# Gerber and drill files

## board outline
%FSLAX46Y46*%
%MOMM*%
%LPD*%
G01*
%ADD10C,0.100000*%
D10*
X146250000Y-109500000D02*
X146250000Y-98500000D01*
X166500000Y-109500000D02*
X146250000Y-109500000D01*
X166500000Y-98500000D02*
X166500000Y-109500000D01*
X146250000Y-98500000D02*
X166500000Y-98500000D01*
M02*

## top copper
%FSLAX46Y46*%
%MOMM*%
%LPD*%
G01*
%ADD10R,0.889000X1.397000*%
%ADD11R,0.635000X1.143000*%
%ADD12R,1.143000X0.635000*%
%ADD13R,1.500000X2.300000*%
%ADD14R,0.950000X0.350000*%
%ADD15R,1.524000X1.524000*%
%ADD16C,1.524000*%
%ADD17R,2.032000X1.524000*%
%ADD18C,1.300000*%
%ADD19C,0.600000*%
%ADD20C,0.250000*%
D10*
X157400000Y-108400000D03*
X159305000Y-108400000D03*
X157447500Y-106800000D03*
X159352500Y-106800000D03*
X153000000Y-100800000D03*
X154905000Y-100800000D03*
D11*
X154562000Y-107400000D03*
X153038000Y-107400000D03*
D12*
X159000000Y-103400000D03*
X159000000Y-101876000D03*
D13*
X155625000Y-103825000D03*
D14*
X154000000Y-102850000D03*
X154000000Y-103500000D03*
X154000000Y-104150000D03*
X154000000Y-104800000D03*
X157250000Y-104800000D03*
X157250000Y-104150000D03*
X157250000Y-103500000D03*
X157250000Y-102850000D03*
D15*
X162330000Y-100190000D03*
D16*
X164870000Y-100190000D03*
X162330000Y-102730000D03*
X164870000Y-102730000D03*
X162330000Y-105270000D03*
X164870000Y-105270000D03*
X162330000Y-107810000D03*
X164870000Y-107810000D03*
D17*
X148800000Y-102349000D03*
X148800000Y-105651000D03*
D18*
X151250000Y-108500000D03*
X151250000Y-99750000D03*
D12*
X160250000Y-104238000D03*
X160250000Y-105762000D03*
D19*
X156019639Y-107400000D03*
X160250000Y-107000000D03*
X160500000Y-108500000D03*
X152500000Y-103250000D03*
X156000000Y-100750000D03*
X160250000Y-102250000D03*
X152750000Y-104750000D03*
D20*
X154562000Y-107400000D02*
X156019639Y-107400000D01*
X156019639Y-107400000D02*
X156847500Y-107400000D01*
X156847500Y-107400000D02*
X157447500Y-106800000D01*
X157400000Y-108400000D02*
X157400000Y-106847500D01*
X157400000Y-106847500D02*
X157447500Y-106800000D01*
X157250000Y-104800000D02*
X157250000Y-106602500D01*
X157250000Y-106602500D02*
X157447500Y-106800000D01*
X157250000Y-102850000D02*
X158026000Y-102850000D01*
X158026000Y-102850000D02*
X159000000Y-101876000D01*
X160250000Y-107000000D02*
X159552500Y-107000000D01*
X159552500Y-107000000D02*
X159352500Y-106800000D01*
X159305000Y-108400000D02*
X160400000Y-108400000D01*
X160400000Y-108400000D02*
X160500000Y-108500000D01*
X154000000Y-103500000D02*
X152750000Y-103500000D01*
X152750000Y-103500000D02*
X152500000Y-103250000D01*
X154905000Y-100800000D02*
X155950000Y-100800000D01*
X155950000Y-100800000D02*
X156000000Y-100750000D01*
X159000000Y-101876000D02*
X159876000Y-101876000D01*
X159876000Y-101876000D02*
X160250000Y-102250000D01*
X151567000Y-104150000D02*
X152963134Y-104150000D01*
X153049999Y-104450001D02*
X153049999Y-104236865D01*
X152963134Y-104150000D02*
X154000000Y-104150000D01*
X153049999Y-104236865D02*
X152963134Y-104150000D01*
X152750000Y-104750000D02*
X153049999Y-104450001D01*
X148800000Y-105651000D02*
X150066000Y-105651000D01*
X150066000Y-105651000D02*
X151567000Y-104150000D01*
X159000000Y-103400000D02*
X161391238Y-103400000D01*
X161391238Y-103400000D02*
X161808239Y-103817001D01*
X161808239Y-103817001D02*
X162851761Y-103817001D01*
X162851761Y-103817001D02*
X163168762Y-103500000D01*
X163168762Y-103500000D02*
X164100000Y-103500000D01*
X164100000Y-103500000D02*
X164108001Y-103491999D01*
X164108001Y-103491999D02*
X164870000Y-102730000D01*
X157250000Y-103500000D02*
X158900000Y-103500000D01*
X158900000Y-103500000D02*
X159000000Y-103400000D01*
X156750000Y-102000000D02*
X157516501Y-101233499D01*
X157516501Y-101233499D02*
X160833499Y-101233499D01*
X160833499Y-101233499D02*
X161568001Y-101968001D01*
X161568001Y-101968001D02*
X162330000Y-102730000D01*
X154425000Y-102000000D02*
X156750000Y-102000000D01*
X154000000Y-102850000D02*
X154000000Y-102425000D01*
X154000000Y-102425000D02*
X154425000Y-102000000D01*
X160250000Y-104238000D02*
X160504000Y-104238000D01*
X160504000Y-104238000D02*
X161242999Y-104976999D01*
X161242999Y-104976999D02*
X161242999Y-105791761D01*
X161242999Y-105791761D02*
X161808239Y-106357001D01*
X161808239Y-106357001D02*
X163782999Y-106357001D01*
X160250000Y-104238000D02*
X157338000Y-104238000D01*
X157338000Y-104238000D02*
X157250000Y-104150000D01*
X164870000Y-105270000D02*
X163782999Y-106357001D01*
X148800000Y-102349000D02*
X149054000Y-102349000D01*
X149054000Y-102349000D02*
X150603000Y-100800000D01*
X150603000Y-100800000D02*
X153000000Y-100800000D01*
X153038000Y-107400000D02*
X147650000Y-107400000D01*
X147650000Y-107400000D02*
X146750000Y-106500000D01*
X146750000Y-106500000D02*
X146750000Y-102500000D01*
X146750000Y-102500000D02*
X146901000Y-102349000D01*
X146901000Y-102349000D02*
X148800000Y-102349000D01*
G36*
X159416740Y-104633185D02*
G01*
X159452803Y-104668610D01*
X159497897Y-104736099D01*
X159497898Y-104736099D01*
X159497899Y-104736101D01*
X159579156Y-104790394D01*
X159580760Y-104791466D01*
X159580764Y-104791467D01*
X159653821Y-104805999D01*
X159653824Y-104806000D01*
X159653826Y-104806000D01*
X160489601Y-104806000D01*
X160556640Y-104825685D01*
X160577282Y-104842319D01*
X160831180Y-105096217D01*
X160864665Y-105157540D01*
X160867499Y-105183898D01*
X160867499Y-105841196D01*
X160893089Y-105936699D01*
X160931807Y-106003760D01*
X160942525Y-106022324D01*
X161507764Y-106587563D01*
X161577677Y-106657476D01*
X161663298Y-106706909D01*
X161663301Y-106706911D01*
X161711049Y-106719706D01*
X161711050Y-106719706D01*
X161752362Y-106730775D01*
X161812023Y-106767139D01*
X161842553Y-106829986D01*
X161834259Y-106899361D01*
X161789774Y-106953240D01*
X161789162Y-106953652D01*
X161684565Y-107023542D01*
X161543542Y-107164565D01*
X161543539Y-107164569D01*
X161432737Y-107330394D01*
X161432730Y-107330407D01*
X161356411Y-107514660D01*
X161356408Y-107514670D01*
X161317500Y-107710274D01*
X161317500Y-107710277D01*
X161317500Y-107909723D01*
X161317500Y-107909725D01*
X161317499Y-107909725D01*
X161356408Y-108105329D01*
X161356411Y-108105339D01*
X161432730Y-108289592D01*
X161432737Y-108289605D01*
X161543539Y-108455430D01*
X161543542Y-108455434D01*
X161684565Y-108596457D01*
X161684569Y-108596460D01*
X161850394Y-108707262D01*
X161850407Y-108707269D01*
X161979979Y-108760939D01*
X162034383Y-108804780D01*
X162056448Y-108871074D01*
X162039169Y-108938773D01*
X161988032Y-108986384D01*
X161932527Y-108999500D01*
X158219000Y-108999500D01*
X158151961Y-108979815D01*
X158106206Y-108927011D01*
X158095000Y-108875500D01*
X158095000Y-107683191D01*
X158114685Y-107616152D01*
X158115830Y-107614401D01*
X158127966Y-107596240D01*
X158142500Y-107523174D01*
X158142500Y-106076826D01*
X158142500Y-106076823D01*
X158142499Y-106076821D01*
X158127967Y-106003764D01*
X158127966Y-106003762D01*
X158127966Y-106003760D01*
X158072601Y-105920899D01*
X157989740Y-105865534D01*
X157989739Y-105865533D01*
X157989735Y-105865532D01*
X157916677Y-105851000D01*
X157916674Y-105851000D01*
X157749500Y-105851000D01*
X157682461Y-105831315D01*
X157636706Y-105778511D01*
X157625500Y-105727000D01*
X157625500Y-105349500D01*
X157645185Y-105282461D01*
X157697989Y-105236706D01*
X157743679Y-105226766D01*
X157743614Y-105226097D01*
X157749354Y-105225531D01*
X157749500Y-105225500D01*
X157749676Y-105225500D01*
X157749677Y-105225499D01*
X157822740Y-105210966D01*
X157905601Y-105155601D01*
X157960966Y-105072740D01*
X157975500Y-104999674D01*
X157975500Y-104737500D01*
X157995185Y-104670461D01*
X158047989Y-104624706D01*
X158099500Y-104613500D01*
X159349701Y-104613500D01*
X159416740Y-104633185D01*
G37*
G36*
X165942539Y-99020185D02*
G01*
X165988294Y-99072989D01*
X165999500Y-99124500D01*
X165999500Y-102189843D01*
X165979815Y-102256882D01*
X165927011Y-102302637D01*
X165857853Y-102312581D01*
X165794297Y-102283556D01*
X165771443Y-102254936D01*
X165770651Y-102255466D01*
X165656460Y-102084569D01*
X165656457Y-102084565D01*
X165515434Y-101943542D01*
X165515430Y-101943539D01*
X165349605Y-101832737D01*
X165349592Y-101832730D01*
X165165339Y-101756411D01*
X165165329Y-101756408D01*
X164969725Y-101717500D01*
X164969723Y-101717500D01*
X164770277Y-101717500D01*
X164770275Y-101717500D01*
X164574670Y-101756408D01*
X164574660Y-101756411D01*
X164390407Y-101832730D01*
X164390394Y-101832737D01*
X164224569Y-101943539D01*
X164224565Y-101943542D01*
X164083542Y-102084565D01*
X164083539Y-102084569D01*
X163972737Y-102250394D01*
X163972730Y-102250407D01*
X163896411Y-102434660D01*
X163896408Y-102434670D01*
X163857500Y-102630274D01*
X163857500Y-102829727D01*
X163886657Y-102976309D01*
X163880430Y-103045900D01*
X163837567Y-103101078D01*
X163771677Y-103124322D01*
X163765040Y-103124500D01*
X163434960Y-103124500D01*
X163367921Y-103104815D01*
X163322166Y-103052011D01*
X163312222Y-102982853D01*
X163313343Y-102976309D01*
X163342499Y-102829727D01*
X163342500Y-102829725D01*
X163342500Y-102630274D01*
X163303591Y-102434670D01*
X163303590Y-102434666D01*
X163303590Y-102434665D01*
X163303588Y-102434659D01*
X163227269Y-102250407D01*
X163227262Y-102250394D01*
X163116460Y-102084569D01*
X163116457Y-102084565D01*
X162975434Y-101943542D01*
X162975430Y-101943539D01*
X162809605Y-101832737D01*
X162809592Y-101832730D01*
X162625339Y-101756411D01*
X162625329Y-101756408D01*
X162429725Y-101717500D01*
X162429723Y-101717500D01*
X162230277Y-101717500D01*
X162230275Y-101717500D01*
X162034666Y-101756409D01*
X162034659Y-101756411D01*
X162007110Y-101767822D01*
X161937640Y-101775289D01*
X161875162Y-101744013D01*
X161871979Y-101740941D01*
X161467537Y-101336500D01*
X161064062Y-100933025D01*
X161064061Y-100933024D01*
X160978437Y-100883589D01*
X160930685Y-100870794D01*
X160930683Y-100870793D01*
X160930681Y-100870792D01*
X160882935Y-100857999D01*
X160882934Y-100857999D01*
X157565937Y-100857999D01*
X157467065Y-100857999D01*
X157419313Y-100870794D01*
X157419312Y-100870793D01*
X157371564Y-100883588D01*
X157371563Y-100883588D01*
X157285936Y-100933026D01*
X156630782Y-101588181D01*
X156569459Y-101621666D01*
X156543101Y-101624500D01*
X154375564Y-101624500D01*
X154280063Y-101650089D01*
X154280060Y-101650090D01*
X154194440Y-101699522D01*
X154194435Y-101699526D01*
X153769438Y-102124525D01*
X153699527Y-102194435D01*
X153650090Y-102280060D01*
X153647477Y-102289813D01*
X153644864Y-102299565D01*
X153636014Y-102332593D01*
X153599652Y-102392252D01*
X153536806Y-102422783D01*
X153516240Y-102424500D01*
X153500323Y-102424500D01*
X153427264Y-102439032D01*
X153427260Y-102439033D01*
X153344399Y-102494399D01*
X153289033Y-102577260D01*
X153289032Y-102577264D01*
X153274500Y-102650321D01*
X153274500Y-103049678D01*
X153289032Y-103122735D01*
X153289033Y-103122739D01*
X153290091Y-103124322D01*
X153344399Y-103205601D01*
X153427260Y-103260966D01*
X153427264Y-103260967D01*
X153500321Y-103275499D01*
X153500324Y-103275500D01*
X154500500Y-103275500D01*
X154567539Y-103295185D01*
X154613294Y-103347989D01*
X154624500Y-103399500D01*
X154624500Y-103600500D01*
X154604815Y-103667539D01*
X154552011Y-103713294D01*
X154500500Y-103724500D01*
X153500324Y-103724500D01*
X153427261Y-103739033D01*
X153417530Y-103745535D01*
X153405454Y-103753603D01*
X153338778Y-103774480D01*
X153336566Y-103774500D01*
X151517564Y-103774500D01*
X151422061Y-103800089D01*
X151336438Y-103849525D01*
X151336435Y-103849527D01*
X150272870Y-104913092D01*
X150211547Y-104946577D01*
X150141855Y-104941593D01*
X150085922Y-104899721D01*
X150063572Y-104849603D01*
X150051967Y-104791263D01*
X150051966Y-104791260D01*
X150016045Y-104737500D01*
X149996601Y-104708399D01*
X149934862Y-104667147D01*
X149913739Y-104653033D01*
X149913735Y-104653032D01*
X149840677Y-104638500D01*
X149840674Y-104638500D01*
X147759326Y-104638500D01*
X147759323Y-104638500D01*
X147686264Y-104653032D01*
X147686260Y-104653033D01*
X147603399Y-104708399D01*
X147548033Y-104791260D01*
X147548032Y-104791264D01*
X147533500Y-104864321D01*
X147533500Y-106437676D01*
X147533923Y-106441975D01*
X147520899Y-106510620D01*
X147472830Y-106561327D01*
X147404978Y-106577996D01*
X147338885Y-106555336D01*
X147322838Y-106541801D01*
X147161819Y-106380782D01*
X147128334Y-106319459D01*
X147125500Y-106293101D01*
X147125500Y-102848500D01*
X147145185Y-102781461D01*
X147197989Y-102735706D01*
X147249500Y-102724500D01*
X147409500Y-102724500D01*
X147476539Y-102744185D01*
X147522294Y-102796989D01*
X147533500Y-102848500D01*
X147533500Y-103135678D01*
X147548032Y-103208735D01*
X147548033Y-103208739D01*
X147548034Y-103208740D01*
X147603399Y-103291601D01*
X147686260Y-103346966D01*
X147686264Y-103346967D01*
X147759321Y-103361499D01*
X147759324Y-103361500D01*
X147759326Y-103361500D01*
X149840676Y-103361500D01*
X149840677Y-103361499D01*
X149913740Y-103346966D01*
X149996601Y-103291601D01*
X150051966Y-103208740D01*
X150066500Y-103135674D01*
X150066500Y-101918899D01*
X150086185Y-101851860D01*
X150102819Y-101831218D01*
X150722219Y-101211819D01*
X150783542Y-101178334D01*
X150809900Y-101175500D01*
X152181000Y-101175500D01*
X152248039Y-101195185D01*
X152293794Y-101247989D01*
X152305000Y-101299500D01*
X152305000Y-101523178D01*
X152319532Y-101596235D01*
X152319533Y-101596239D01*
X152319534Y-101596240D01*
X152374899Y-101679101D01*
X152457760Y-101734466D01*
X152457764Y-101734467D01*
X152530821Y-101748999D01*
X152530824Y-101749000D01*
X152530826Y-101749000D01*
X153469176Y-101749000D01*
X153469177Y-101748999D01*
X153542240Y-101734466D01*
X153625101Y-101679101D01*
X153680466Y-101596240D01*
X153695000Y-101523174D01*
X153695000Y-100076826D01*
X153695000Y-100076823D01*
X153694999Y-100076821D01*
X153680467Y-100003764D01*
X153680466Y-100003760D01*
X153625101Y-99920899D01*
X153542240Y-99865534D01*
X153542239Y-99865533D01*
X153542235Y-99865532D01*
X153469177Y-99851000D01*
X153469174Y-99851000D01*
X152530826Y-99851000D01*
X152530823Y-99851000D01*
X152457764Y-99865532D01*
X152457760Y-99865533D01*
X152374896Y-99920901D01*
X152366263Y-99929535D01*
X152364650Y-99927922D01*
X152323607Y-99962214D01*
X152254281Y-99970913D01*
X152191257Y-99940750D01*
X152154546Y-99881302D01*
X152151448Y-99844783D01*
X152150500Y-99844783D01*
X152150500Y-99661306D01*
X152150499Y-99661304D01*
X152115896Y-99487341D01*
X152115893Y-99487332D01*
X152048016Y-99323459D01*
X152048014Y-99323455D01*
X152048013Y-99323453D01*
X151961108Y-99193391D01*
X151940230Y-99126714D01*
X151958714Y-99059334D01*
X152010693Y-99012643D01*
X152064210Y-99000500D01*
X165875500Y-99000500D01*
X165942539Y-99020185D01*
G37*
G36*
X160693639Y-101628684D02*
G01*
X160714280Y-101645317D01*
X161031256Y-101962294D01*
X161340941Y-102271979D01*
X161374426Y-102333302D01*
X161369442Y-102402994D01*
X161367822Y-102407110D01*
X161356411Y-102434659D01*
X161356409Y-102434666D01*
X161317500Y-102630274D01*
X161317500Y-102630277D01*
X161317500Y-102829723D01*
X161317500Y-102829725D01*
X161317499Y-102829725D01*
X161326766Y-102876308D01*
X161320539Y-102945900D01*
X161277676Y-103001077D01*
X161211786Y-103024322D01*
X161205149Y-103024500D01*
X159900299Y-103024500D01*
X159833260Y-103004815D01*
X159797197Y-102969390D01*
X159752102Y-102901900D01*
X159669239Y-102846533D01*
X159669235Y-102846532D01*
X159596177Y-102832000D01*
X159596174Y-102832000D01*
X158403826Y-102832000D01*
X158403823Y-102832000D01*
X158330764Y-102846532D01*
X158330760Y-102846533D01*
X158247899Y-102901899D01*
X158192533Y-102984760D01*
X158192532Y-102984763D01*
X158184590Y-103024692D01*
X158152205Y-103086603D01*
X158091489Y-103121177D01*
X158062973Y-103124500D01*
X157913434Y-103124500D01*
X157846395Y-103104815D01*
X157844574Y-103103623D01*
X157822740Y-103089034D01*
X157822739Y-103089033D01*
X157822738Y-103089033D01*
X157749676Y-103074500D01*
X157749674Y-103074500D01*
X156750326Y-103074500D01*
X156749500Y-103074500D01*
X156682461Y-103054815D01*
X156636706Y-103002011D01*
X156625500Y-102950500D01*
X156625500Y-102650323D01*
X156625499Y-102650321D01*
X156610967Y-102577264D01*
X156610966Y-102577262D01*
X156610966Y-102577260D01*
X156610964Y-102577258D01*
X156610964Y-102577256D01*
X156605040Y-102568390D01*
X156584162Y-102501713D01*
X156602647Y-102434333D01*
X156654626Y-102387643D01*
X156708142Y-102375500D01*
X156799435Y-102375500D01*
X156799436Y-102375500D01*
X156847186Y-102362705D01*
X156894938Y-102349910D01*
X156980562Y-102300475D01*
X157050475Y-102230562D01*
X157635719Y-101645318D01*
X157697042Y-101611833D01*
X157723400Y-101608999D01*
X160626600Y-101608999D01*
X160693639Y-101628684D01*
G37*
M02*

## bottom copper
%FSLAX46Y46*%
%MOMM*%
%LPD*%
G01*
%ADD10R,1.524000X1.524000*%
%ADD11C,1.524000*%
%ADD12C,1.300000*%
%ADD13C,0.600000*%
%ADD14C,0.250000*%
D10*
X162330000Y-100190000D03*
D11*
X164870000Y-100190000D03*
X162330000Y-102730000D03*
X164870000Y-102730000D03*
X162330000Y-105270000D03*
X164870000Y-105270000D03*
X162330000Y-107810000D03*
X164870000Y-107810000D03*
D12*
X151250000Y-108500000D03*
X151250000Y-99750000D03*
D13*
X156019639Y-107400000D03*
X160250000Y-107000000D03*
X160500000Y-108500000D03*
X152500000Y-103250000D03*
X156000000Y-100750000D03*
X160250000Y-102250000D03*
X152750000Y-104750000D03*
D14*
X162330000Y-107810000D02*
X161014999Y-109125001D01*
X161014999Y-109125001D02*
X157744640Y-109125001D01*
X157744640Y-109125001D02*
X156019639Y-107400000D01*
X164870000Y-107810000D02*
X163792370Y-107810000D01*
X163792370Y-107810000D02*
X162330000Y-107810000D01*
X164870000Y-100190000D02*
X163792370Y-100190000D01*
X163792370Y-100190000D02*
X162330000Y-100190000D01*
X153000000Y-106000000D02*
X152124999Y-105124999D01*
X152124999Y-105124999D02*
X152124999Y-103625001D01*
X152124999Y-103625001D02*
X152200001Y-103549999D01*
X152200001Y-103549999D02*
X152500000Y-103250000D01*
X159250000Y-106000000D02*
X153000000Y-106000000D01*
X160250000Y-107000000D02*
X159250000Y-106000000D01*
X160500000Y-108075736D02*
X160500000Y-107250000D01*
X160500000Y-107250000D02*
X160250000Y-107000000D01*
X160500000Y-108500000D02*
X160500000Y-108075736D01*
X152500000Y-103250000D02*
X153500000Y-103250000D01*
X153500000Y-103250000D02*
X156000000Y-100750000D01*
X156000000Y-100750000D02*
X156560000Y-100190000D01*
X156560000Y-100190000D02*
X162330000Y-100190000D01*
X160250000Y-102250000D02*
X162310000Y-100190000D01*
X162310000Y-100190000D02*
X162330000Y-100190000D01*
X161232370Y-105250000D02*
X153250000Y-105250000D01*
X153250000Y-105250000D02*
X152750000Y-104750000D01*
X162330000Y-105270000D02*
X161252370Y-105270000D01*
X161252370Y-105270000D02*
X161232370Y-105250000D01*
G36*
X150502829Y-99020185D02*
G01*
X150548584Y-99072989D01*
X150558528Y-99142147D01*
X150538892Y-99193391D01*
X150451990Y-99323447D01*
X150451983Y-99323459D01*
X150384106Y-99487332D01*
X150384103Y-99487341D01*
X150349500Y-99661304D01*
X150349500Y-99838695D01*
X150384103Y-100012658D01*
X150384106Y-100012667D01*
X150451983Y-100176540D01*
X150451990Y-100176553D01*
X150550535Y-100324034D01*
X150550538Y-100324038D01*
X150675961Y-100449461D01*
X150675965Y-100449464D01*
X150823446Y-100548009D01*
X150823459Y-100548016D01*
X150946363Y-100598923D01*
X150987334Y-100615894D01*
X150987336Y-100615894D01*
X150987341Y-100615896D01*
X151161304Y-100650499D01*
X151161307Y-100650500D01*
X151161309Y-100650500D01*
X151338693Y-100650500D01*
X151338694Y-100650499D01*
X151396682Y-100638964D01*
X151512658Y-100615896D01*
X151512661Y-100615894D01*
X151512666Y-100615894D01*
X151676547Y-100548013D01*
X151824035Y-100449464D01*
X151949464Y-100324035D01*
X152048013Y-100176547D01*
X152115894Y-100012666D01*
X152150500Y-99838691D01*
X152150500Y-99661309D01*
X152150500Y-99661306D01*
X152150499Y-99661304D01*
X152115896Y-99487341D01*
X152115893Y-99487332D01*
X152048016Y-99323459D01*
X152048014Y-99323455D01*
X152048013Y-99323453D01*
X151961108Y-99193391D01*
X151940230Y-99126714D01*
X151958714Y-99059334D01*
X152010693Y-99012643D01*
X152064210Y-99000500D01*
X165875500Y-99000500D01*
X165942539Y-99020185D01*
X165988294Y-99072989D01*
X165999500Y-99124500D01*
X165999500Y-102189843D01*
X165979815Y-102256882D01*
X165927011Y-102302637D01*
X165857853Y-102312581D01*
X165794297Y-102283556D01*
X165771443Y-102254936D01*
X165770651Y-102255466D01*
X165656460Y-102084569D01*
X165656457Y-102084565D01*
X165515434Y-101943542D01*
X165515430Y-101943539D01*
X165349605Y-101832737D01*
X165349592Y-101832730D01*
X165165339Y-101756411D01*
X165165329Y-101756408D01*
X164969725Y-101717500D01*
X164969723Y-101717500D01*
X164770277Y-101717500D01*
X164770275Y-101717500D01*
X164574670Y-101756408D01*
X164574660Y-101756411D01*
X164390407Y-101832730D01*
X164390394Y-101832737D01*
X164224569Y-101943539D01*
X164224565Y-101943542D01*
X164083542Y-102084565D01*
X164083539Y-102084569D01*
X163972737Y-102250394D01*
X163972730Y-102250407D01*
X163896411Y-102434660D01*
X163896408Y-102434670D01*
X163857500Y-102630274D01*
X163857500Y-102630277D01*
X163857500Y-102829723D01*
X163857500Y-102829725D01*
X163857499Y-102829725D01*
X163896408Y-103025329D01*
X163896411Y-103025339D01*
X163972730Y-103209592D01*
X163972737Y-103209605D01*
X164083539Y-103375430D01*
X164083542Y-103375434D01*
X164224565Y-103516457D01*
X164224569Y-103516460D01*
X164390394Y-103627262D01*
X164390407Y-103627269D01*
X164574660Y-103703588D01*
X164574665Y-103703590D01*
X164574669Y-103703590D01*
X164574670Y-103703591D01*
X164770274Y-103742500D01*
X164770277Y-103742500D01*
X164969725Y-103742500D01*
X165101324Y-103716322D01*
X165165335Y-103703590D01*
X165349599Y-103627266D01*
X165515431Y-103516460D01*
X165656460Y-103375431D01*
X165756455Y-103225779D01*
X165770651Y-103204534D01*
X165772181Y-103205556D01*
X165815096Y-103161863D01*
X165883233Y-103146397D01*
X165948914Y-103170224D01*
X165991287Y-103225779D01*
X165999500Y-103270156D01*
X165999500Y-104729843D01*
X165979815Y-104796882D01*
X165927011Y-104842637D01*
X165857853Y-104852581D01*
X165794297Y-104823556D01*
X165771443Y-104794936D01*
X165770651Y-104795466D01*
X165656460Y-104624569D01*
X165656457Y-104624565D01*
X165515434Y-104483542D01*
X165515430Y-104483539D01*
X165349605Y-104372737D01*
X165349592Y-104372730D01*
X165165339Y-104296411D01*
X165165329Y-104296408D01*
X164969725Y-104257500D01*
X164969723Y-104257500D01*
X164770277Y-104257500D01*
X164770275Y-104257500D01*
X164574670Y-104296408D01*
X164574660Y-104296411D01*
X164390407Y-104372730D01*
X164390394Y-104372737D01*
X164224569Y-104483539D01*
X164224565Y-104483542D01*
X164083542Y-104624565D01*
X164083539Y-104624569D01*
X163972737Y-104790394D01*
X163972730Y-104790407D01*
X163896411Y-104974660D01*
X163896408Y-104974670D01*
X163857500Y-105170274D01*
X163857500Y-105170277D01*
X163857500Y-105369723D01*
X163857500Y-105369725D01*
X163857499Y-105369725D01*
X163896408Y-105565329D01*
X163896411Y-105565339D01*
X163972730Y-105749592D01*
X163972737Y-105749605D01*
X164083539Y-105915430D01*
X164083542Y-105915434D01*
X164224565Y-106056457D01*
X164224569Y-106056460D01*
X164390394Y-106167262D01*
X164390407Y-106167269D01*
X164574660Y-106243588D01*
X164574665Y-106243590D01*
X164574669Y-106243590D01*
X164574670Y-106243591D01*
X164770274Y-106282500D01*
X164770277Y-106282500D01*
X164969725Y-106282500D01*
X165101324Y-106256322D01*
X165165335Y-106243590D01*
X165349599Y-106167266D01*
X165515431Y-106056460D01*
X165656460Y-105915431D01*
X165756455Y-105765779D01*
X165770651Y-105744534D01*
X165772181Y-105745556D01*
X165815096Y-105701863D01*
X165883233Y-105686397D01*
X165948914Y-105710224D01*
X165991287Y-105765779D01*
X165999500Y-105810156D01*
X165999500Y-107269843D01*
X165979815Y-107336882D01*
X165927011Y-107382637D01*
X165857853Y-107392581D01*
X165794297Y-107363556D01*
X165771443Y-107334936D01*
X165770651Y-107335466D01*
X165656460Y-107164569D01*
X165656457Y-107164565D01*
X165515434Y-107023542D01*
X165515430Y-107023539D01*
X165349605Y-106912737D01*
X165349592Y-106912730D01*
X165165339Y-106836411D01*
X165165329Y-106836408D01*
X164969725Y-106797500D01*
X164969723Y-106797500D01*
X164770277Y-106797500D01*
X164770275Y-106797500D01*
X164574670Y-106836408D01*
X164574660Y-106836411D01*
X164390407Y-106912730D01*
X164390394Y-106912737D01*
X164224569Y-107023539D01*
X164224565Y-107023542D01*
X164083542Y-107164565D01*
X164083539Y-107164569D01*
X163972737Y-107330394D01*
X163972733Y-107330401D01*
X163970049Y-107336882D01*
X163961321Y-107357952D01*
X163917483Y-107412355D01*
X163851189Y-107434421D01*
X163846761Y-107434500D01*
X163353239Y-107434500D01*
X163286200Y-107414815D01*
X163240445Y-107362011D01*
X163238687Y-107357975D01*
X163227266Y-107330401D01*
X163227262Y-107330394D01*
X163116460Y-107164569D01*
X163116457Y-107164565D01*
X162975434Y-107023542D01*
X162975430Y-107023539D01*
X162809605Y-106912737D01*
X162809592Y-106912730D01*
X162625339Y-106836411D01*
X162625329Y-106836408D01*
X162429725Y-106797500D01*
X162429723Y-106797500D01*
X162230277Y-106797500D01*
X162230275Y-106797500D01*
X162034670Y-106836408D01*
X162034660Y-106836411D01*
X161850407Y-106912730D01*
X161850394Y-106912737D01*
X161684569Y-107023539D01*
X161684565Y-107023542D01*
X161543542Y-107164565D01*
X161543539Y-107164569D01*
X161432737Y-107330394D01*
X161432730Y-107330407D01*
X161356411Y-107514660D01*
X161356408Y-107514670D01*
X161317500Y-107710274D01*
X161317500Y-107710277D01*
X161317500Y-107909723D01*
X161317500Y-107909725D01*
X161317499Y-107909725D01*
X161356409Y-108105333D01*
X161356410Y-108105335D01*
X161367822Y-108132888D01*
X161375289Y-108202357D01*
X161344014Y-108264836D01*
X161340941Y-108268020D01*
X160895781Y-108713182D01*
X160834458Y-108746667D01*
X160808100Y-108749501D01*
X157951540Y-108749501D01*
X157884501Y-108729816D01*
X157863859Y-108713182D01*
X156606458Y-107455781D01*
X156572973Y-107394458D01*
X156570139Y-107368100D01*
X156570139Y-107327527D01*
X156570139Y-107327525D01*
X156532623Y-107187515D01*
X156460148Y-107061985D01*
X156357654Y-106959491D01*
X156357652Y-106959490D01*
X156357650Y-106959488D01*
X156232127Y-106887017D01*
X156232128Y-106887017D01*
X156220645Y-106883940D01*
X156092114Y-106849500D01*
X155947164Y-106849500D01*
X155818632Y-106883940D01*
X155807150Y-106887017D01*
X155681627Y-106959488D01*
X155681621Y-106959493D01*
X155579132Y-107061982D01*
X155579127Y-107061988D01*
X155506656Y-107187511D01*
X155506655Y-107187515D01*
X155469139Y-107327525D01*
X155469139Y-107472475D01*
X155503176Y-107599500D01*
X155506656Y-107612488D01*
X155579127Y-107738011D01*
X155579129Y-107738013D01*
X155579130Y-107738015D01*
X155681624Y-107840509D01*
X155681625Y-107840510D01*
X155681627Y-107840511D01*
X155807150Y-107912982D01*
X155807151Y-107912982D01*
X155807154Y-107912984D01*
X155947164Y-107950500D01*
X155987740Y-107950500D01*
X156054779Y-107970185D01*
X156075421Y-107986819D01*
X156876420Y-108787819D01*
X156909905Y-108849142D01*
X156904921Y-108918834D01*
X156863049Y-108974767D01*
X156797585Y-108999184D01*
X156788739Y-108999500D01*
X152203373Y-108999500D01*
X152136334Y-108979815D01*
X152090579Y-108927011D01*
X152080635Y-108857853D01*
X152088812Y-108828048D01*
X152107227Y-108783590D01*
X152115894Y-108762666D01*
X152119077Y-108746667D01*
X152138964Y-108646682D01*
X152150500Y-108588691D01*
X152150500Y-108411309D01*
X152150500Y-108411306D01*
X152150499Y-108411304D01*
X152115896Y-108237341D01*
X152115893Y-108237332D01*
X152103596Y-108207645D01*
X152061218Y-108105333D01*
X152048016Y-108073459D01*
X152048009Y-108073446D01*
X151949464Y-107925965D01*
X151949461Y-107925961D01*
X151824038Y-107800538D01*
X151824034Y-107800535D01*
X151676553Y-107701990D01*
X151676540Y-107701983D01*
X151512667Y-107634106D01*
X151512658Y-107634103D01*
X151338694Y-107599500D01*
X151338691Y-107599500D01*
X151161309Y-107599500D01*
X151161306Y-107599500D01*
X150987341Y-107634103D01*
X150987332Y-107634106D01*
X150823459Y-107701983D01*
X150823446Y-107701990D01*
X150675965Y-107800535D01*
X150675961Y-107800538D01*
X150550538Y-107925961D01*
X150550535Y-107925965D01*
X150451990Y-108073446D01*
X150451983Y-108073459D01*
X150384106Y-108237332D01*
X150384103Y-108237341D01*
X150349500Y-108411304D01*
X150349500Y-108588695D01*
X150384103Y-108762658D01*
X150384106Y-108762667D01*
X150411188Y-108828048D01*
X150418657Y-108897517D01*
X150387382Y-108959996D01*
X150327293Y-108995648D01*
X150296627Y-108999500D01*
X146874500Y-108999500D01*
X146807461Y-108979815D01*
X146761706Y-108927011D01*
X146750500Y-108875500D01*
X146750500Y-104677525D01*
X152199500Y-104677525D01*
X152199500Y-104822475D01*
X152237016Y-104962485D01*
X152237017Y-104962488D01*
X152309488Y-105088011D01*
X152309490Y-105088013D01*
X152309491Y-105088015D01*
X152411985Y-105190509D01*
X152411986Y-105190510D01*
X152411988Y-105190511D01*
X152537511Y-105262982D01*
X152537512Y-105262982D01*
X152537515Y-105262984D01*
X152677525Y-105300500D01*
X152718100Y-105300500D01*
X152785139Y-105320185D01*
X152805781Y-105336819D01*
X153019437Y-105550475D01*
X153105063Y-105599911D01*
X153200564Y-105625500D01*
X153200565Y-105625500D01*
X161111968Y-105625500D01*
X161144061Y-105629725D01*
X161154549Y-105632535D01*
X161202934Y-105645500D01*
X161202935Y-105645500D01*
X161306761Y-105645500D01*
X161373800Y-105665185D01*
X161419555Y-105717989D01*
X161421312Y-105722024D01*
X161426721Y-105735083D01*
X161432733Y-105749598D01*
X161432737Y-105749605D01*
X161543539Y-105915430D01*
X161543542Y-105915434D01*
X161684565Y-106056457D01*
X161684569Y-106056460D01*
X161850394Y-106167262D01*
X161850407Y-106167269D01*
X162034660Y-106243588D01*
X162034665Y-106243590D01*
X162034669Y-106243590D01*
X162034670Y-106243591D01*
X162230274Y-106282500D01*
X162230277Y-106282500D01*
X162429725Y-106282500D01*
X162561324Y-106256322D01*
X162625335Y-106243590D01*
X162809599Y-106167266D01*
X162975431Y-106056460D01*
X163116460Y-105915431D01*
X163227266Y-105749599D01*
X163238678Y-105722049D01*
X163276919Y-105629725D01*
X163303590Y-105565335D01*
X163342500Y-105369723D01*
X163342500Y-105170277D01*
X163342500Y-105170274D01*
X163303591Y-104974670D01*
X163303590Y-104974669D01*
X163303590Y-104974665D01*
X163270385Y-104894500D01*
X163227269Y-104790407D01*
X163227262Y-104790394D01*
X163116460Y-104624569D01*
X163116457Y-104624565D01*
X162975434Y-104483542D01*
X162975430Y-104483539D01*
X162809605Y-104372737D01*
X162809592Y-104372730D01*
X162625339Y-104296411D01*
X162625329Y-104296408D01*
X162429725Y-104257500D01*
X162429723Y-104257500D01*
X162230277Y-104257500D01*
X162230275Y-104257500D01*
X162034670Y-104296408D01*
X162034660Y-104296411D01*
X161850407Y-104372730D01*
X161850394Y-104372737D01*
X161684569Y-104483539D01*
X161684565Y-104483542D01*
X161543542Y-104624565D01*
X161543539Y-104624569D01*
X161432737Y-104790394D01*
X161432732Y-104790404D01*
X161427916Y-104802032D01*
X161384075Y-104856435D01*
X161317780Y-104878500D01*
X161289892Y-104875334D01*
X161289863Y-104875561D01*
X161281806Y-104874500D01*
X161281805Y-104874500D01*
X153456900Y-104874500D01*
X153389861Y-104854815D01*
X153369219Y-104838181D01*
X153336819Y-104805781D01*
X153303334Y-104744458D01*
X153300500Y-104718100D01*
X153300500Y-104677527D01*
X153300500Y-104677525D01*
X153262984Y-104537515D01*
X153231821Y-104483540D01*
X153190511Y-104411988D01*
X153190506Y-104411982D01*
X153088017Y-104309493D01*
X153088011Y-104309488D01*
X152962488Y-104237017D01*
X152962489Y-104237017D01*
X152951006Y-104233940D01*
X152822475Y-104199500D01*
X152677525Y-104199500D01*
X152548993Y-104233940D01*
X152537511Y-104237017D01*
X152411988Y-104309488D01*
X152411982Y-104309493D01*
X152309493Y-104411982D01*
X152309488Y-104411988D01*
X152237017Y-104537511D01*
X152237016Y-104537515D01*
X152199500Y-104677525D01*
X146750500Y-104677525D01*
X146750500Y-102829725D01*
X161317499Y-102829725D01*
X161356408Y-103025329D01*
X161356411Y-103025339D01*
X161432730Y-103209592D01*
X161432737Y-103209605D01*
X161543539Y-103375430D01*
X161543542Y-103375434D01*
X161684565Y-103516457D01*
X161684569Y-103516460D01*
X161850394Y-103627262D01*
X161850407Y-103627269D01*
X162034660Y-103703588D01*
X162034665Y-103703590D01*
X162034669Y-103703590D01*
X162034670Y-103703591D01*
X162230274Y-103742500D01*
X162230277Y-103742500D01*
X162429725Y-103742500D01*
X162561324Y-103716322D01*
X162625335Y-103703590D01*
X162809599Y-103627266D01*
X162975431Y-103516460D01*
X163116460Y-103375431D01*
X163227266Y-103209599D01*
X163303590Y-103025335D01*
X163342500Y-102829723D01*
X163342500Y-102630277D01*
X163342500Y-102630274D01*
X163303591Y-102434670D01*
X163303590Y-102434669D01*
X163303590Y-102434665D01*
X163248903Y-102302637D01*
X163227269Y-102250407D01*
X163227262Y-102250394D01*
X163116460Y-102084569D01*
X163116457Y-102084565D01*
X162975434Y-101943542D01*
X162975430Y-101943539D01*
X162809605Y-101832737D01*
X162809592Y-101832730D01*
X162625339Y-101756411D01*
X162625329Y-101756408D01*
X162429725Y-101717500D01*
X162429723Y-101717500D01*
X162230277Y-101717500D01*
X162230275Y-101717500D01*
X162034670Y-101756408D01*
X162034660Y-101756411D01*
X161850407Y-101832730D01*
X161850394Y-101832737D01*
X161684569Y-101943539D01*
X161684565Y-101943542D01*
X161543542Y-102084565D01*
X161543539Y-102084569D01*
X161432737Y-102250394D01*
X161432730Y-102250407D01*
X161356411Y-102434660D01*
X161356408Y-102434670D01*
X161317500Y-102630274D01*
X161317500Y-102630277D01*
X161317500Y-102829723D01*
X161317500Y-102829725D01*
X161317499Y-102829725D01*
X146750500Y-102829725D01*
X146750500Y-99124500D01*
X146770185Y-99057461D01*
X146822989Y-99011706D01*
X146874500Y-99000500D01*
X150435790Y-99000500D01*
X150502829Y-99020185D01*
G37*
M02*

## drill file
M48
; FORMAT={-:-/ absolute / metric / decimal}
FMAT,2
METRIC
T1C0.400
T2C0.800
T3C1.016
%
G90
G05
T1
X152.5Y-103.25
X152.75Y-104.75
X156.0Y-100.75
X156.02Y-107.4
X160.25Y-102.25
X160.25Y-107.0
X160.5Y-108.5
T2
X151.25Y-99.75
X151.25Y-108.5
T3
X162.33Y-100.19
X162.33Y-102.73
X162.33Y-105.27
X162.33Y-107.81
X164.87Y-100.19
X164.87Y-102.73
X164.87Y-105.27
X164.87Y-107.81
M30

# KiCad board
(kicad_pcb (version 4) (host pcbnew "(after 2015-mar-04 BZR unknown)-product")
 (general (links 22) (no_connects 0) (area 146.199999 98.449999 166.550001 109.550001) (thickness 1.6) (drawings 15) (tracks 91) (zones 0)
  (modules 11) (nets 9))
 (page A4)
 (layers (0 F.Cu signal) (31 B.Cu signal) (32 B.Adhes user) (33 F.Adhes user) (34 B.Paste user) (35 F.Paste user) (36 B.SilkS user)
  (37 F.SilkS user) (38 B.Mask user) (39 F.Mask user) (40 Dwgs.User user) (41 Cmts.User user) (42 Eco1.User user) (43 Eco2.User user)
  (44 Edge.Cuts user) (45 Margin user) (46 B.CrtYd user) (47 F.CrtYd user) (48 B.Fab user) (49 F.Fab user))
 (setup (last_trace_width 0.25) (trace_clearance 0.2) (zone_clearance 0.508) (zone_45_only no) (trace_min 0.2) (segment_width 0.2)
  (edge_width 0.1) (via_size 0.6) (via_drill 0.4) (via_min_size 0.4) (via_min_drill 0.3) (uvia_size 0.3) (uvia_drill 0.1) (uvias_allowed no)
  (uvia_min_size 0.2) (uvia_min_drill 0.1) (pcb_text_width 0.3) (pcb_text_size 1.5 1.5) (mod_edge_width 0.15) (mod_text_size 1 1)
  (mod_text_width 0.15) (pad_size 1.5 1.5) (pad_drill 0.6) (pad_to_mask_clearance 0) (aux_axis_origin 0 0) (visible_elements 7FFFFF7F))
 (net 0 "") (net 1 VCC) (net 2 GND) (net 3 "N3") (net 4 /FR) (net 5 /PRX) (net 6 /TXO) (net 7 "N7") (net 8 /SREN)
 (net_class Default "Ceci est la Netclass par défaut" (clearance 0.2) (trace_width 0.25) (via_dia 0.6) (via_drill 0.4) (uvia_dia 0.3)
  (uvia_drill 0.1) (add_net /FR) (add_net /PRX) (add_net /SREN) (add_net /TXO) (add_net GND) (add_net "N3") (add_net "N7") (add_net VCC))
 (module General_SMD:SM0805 (layer F.Cu) (at 158.3525 108.4)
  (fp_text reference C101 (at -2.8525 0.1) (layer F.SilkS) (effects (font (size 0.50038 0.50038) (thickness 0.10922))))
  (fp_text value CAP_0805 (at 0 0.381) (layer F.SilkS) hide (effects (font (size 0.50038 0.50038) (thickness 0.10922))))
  (pad 1 smd rect (at -0.9525 0) (size 0.889 1.397) (layers F.Cu F.Paste F.Mask) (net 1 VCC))
  (pad 2 smd rect (at 0.9525 0) (size 0.889 1.397) (layers F.Cu F.Paste F.Mask) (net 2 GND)))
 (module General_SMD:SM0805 (layer F.Cu) (at 158.4 106.8)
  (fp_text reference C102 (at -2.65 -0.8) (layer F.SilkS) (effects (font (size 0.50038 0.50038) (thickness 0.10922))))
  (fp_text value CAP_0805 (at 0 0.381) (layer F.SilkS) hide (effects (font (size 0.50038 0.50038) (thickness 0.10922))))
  (pad 1 smd rect (at -0.9525 0) (size 0.889 1.397) (layers F.Cu F.Paste F.Mask) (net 1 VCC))
  (pad 2 smd rect (at 0.9525 0) (size 0.889 1.397) (layers F.Cu F.Paste F.Mask) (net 2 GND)))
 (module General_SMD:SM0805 (layer F.Cu) (at 153.9525 100.8)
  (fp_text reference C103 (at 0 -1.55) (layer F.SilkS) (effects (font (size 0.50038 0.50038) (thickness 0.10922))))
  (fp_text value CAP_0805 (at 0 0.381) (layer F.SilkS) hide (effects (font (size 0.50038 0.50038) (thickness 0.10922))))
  (pad 1 smd rect (at -0.9525 0) (size 0.889 1.397) (layers F.Cu F.Paste F.Mask) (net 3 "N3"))
  (pad 2 smd rect (at 0.9525 0) (size 0.889 1.397) (layers F.Cu F.Paste F.Mask) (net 2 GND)))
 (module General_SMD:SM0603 (layer F.Cu) (at 153.8 107.4 180)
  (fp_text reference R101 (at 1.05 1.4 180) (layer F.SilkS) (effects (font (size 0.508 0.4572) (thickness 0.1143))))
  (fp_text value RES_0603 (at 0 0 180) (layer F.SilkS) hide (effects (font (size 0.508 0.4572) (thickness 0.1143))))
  (pad 1 smd rect (at -0.762 0 180) (size 0.635 1.143) (layers F.Cu F.Paste F.Mask) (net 1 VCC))
  (pad 2 smd rect (at 0.762 0 180) (size 0.635 1.143) (layers F.Cu F.Paste F.Mask) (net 3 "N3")))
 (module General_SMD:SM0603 (layer F.Cu) (at 159 102.638 90)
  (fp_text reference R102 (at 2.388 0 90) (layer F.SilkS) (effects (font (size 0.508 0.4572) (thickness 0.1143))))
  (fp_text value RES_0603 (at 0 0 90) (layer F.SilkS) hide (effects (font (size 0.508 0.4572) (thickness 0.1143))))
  (pad 1 smd rect (at -0.762 0 90) (size 0.635 1.143) (layers F.Cu F.Paste F.Mask) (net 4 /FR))
  (pad 2 smd rect (at 0.762 0 90) (size 0.635 1.143) (layers F.Cu F.Paste F.Mask) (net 2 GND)))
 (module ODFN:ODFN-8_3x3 (layer F.Cu) (at 155.625 103.825 270)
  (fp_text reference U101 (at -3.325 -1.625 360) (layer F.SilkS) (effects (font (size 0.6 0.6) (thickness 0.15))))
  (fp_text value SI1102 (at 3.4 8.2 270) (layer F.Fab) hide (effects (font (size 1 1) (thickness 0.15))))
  (pad 9 smd rect (at 0 0 270) (size 2.3 1.5) (layers F.Cu F.Paste F.Mask))
  (pad 1 smd rect (at -0.975 1.625 270) (size 0.35 0.95) (layers F.Cu F.Paste F.Mask) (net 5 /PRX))
  (pad 2 smd rect (at -0.325 1.625 270) (size 0.35 0.95) (layers F.Cu F.Paste F.Mask) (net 2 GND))
  (pad 3 smd rect (at 0.325 1.625 270) (size 0.35 0.95) (layers F.Cu F.Paste F.Mask) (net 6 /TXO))
  (pad 4 smd rect (at 0.975 1.625 270) (size 0.35 0.95) (layers F.Cu F.Paste F.Mask) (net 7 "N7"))
  (pad 5 smd rect (at 0.975 -1.625 270) (size 0.35 0.95) (layers F.Cu F.Paste F.Mask) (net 1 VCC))
  (pad 6 smd rect (at 0.325 -1.625 270) (size 0.35 0.95) (layers F.Cu F.Paste F.Mask) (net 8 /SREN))
  (pad 7 smd rect (at -0.325 -1.625 270) (size 0.35 0.95) (layers F.Cu F.Paste F.Mask) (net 4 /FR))
  (pad 8 smd rect (at -0.975 -1.625 270) (size 0.35 0.95) (layers F.Cu F.Paste F.Mask) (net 2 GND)))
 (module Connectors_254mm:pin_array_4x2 (layer F.Cu) (at 163.6 104 270)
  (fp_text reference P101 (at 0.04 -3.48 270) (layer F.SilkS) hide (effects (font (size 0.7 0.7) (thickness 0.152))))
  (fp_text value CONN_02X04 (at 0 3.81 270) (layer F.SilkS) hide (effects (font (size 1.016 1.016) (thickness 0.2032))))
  (pad 1 thru_hole rect (at -3.81 1.27 270) (size 1.524 1.524) (drill 1.016) (layers *.Cu *.Mask F.SilkS) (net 2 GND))
  (pad 2 thru_hole circle (at -3.81 -1.27 270) (size 1.524 1.524) (drill 1.016) (layers *.Cu *.Mask F.SilkS) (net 2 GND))
  (pad 3 thru_hole circle (at -1.27 1.27 270) (size 1.524 1.524) (drill 1.016) (layers *.Cu *.Mask F.SilkS) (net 5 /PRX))
  (pad 4 thru_hole circle (at -1.27 -1.27 270) (size 1.524 1.524) (drill 1.016) (layers *.Cu *.Mask F.SilkS) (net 4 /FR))
  (pad 5 thru_hole circle (at 1.27 1.27 270) (size 1.524 1.524) (drill 1.016) (layers *.Cu *.Mask F.SilkS) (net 6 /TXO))
  (pad 6 thru_hole circle (at 1.27 -1.27 270) (size 1.524 1.524) (drill 1.016) (layers *.Cu *.Mask F.SilkS) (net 8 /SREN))
  (pad 7 thru_hole circle (at 3.81 1.27 270) (size 1.524 1.524) (drill 1.016) (layers *.Cu *.Mask F.SilkS) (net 1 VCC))
  (pad 8 thru_hole circle (at 3.81 -1.27 270) (size 1.524 1.524) (drill 1.016) (layers *.Cu *.Mask F.SilkS) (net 1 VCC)))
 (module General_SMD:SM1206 (layer F.Cu) (at 148.8 104 270)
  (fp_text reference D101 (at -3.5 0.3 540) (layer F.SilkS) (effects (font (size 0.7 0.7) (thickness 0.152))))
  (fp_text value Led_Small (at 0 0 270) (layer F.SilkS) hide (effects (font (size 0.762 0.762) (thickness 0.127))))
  (pad 1 smd rect (at -1.651 0 270) (size 1.524 2.032) (layers F.Cu F.Paste F.Mask) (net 3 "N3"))
  (pad 2 smd rect (at 1.651 0 270) (size 1.524 2.032) (layers F.Cu F.Paste F.Mask) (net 6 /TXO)))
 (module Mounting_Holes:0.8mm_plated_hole (layer F.Cu) (at 151.25 108.5)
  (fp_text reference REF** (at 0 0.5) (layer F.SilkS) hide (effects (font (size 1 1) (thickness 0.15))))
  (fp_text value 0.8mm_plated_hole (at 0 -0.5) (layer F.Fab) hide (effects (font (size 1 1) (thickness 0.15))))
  (pad 1 thru_hole circle (at 0 0) (size 1.3 1.3) (drill 0.8) (layers *.Cu *.SilkS *.Mask)))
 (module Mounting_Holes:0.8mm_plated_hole (layer F.Cu) (at 151.25 99.75)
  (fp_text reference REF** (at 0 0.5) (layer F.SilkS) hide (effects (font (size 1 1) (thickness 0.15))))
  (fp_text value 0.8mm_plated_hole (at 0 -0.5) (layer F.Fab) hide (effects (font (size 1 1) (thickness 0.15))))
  (pad 1 thru_hole circle (at 0 0) (size 1.3 1.3) (drill 0.8) (layers *.Cu *.SilkS *.Mask)))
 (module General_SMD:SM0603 (layer F.Cu) (at 160.25 105 270)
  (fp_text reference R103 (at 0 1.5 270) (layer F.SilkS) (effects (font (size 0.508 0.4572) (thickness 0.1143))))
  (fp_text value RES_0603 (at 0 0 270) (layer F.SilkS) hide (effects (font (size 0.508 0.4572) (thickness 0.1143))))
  (pad 1 smd rect (at -0.762 0 270) (size 0.635 1.143) (layers F.Cu F.Paste F.Mask) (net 8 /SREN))
  (pad 2 smd rect (at 0.762 0 270) (size 0.635 1.143) (layers F.Cu F.Paste F.Mask) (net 2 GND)))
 (gr_line (start 146.25 109.5) (end 146.25 98.5) (layer Edge.Cuts) (width 0.1))
 (gr_line (start 166.5 109.5) (end 146.25 109.5) (layer Edge.Cuts) (width 0.1))
 (gr_line (start 166.5 98.5) (end 166.5 109.5) (layer Edge.Cuts) (width 0.1))
 (gr_line (start 146.25 98.5) (end 166.5 98.5) (layer Edge.Cuts) (width 0.1))
 (segment (start 154.562 107.4) (end 156.019639 107.4) (width 0.25) (layer F.Cu) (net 1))
 (segment (start 156.019639 107.4) (end 156.8475 107.4) (width 0.25) (layer F.Cu) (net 1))
 (via (at 156.019639 107.4) (size 0.6) (drill 0.4) (layers F.Cu B.Cu) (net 1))
 (segment (start 162.33 107.81) (end 161.014999 109.125001) (width 0.25) (layer B.Cu) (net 1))
 (segment (start 161.014999 109.125001) (end 157.74464 109.125001) (width 0.25) (layer B.Cu) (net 1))
 (segment (start 157.74464 109.125001) (end 156.019639 107.4) (width 0.25) (layer B.Cu) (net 1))
 (segment (start 164.87 107.81) (end 163.79237 107.81) (width 0.25) (layer B.Cu) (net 1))
 (segment (start 163.79237 107.81) (end 162.33 107.81) (width 0.25) (layer B.Cu) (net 1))
 (segment (start 156.8475 107.4) (end 157.4475 106.8) (width 0.25) (layer F.Cu) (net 1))
 (segment (start 157.4 108.4) (end 157.4 106.8475) (width 0.25) (layer F.Cu) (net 1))
 (segment (start 157.4 106.8475) (end 157.4475 106.8) (width 0.25) (layer F.Cu) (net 1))
 (segment (start 157.25 104.8) (end 157.25 106.6025) (width 0.25) (layer F.Cu) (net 1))
 (segment (start 157.25 106.6025) (end 157.4475 106.8) (width 0.25) (layer F.Cu) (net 1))
 (segment (start 164.87 100.19) (end 163.79237 100.19) (width 0.25) (layer B.Cu) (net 2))
 (segment (start 163.79237 100.19) (end 162.33 100.19) (width 0.25) (layer B.Cu) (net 2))
 (segment (start 153 106) (end 152.124999 105.124999) (width 0.25) (layer B.Cu) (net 2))
 (segment (start 152.124999 105.124999) (end 152.124999 103.625001) (width 0.25) (layer B.Cu) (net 2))
 (segment (start 152.124999 103.625001) (end 152.200001 103.549999) (width 0.25) (layer B.Cu) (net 2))
 (segment (start 152.200001 103.549999) (end 152.5 103.25) (width 0.25) (layer B.Cu) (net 2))
 (segment (start 159.25 106) (end 153 106) (width 0.25) (layer B.Cu) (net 2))
 (segment (start 160.25 107) (end 159.25 106) (width 0.25) (layer B.Cu) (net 2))
 (segment (start 157.25 102.85) (end 158.026 102.85) (width 0.25) (layer F.Cu) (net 2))
 (segment (start 158.026 102.85) (end 159 101.876) (width 0.25) (layer F.Cu) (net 2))
 (segment (start 160.25 107) (end 159.5525 107) (width 0.25) (layer F.Cu) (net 2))
 (segment (start 159.5525 107) (end 159.3525 106.8) (width 0.25) (layer F.Cu) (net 2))
 (segment (start 160.5 108.075736) (end 160.5 107.25) (width 0.25) (layer B.Cu) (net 2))
 (segment (start 160.5 107.25) (end 160.25 107) (width 0.25) (layer B.Cu) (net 2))
 (via (at 160.25 107) (size 0.6) (drill 0.4) (layers F.Cu B.Cu) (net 2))
 (segment (start 160.5 108.5) (end 160.5 108.075736) (width 0.25) (layer B.Cu) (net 2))
 (segment (start 159.305 108.4) (end 160.4 108.4) (width 0.25) (layer F.Cu) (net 2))
 (segment (start 160.4 108.4) (end 160.5 108.5) (width 0.25) (layer F.Cu) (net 2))
 (via (at 160.5 108.5) (size 0.6) (drill 0.4) (layers F.Cu B.Cu) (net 2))
 (segment (start 152.5 103.25) (end 153.5 103.25) (width 0.25) (layer B.Cu) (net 2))
 (segment (start 153.5 103.25) (end 156 100.75) (width 0.25) (layer B.Cu) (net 2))
 (segment (start 156 100.75) (end 156.56 100.19) (width 0.25) (layer B.Cu) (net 2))
 (segment (start 156.56 100.19) (end 162.33 100.19) (width 0.25) (layer B.Cu) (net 2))
 (segment (start 160.25 102.25) (end 162.31 100.19) (width 0.25) (layer B.Cu) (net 2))
 (segment (start 162.31 100.19) (end 162.33 100.19) (width 0.25) (layer B.Cu) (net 2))
 (segment (start 154 103.5) (end 152.75 103.5) (width 0.25) (layer F.Cu) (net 2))
 (segment (start 152.75 103.5) (end 152.5 103.25) (width 0.25) (layer F.Cu) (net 2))
 (via (at 152.5 103.25) (size 0.6) (drill 0.4) (layers F.Cu B.Cu) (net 2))
 (segment (start 154.905 100.8) (end 155.95 100.8) (width 0.25) (layer F.Cu) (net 2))
 (segment (start 155.95 100.8) (end 156 100.75) (width 0.25) (layer F.Cu) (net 2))
 (via (at 156 100.75) (size 0.6) (drill 0.4) (layers F.Cu B.Cu) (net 2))
 (segment (start 159 101.876) (end 159.876 101.876) (width 0.25) (layer F.Cu) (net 2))
 (segment (start 159.876 101.876) (end 160.25 102.25) (width 0.25) (layer F.Cu) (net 2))
 (via (at 160.25 102.25) (size 0.6) (drill 0.4) (layers F.Cu B.Cu) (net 2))
 (segment (start 151.567 104.15) (end 152.963134 104.15) (width 0.25) (layer F.Cu) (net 6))
 (segment (start 153.049999 104.450001) (end 153.049999 104.236865) (width 0.25) (layer F.Cu) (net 6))
 (segment (start 152.963134 104.15) (end 154 104.15) (width 0.25) (layer F.Cu) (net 6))
 (segment (start 153.049999 104.236865) (end 152.963134 104.15) (width 0.25) (layer F.Cu) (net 6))
 (segment (start 152.75 104.75) (end 153.049999 104.450001) (width 0.25) (layer F.Cu) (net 6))
 (segment (start 161.23237 105.25) (end 153.25 105.25) (width 0.25) (layer B.Cu) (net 6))
 (segment (start 153.25 105.25) (end 152.75 104.75) (width 0.25) (layer B.Cu) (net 6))
 (via (at 152.75 104.75) (size 0.6) (drill 0.4) (layers F.Cu B.Cu) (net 6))
 (segment (start 162.33 105.27) (end 161.25237 105.27) (width 0.25) (layer B.Cu) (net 6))
 (segment (start 161.25237 105.27) (end 161.23237 105.25) (width 0.25) (layer B.Cu) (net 6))
 (segment (start 148.8 105.651) (end 150.066 105.651) (width 0.25) (layer F.Cu) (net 6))
 (segment (start 150.066 105.651) (end 151.567 104.15) (width 0.25) (layer F.Cu) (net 6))
 (segment (start 159 103.4) (end 161.391238 103.4) (width 0.25) (layer F.Cu) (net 4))
 (segment (start 161.391238 103.4) (end 161.808239 103.817001) (width 0.25) (layer F.Cu) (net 4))
 (segment (start 161.808239 103.817001) (end 162.851761 103.817001) (width 0.25) (layer F.Cu) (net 4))
 (segment (start 162.851761 103.817001) (end 163.168762 103.5) (width 0.25) (layer F.Cu) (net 4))
 (segment (start 163.168762 103.5) (end 164.1 103.5) (width 0.25) (layer F.Cu) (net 4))
 (segment (start 164.1 103.5) (end 164.108001 103.491999) (width 0.25) (layer F.Cu) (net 4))
 (segment (start 164.108001 103.491999) (end 164.87 102.73) (width 0.25) (layer F.Cu) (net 4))
 (segment (start 157.25 103.5) (end 158.9 103.5) (width 0.25) (layer F.Cu) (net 4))
 (segment (start 158.9 103.5) (end 159 103.4) (width 0.25) (layer F.Cu) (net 4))
 (segment (start 156.75 102) (end 157.516501 101.233499) (width 0.25) (layer F.Cu) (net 5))
 (segment (start 157.516501 101.233499) (end 160.833499 101.233499) (width 0.25) (layer F.Cu) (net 5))
 (segment (start 160.833499 101.233499) (end 161.568001 101.968001) (width 0.25) (layer F.Cu) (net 5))
 (segment (start 161.568001 101.968001) (end 162.33 102.73) (width 0.25) (layer F.Cu) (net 5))
 (segment (start 154.425 102) (end 156.75 102) (width 0.25) (layer F.Cu) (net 5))
 (segment (start 154 102.85) (end 154 102.425) (width 0.25) (layer F.Cu) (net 5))
 (segment (start 154 102.425) (end 154.425 102) (width 0.25) (layer F.Cu) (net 5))
 (segment (start 160.25 104.238) (end 160.504 104.238) (width 0.25) (layer F.Cu) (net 8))
 (segment (start 160.504 104.238) (end 161.242999 104.976999) (width 0.25) (layer F.Cu) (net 8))
 (segment (start 161.242999 104.976999) (end 161.242999 105.791761) (width 0.25) (layer F.Cu) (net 8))
 (segment (start 161.242999 105.791761) (end 161.808239 106.357001) (width 0.25) (layer F.Cu) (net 8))
 (segment (start 161.808239 106.357001) (end 163.782999 106.357001) (width 0.25) (layer F.Cu) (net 8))
 (segment (start 160.25 104.238) (end 157.338 104.238) (width 0.25) (layer F.Cu) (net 8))
 (segment (start 157.338 104.238) (end 157.25 104.15) (width 0.25) (layer F.Cu) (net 8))
 (segment (start 164.87 105.27) (end 163.782999 106.357001) (width 0.25) (layer F.Cu) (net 8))
 (segment (start 148.8 102.349) (end 149.054 102.349) (width 0.25) (layer F.Cu) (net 3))
 (segment (start 149.054 102.349) (end 150.603 100.8) (width 0.25) (layer F.Cu) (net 3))
 (segment (start 150.603 100.8) (end 153 100.8) (width 0.25) (layer F.Cu) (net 3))
 (segment (start 153.038 107.4) (end 147.65 107.4) (width 0.25) (layer F.Cu) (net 3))
 (segment (start 147.65 107.4) (end 146.75 106.5) (width 0.25) (layer F.Cu) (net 3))
 (segment (start 146.75 106.5) (end 146.75 102.5) (width 0.25) (layer F.Cu) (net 3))
 (segment (start 146.75 102.5) (end 146.901 102.349) (width 0.25) (layer F.Cu) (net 3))
 (segment (start 146.901 102.349) (end 148.8 102.349) (width 0.25) (layer F.Cu) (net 3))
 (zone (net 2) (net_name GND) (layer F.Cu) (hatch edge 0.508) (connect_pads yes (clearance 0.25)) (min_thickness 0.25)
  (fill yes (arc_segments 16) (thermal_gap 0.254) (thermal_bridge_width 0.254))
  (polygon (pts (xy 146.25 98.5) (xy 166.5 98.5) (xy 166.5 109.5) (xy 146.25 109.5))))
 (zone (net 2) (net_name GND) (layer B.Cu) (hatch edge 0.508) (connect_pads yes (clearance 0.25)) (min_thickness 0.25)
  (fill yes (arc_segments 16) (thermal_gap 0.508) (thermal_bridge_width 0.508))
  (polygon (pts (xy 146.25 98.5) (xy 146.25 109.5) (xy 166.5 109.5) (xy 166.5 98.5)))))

